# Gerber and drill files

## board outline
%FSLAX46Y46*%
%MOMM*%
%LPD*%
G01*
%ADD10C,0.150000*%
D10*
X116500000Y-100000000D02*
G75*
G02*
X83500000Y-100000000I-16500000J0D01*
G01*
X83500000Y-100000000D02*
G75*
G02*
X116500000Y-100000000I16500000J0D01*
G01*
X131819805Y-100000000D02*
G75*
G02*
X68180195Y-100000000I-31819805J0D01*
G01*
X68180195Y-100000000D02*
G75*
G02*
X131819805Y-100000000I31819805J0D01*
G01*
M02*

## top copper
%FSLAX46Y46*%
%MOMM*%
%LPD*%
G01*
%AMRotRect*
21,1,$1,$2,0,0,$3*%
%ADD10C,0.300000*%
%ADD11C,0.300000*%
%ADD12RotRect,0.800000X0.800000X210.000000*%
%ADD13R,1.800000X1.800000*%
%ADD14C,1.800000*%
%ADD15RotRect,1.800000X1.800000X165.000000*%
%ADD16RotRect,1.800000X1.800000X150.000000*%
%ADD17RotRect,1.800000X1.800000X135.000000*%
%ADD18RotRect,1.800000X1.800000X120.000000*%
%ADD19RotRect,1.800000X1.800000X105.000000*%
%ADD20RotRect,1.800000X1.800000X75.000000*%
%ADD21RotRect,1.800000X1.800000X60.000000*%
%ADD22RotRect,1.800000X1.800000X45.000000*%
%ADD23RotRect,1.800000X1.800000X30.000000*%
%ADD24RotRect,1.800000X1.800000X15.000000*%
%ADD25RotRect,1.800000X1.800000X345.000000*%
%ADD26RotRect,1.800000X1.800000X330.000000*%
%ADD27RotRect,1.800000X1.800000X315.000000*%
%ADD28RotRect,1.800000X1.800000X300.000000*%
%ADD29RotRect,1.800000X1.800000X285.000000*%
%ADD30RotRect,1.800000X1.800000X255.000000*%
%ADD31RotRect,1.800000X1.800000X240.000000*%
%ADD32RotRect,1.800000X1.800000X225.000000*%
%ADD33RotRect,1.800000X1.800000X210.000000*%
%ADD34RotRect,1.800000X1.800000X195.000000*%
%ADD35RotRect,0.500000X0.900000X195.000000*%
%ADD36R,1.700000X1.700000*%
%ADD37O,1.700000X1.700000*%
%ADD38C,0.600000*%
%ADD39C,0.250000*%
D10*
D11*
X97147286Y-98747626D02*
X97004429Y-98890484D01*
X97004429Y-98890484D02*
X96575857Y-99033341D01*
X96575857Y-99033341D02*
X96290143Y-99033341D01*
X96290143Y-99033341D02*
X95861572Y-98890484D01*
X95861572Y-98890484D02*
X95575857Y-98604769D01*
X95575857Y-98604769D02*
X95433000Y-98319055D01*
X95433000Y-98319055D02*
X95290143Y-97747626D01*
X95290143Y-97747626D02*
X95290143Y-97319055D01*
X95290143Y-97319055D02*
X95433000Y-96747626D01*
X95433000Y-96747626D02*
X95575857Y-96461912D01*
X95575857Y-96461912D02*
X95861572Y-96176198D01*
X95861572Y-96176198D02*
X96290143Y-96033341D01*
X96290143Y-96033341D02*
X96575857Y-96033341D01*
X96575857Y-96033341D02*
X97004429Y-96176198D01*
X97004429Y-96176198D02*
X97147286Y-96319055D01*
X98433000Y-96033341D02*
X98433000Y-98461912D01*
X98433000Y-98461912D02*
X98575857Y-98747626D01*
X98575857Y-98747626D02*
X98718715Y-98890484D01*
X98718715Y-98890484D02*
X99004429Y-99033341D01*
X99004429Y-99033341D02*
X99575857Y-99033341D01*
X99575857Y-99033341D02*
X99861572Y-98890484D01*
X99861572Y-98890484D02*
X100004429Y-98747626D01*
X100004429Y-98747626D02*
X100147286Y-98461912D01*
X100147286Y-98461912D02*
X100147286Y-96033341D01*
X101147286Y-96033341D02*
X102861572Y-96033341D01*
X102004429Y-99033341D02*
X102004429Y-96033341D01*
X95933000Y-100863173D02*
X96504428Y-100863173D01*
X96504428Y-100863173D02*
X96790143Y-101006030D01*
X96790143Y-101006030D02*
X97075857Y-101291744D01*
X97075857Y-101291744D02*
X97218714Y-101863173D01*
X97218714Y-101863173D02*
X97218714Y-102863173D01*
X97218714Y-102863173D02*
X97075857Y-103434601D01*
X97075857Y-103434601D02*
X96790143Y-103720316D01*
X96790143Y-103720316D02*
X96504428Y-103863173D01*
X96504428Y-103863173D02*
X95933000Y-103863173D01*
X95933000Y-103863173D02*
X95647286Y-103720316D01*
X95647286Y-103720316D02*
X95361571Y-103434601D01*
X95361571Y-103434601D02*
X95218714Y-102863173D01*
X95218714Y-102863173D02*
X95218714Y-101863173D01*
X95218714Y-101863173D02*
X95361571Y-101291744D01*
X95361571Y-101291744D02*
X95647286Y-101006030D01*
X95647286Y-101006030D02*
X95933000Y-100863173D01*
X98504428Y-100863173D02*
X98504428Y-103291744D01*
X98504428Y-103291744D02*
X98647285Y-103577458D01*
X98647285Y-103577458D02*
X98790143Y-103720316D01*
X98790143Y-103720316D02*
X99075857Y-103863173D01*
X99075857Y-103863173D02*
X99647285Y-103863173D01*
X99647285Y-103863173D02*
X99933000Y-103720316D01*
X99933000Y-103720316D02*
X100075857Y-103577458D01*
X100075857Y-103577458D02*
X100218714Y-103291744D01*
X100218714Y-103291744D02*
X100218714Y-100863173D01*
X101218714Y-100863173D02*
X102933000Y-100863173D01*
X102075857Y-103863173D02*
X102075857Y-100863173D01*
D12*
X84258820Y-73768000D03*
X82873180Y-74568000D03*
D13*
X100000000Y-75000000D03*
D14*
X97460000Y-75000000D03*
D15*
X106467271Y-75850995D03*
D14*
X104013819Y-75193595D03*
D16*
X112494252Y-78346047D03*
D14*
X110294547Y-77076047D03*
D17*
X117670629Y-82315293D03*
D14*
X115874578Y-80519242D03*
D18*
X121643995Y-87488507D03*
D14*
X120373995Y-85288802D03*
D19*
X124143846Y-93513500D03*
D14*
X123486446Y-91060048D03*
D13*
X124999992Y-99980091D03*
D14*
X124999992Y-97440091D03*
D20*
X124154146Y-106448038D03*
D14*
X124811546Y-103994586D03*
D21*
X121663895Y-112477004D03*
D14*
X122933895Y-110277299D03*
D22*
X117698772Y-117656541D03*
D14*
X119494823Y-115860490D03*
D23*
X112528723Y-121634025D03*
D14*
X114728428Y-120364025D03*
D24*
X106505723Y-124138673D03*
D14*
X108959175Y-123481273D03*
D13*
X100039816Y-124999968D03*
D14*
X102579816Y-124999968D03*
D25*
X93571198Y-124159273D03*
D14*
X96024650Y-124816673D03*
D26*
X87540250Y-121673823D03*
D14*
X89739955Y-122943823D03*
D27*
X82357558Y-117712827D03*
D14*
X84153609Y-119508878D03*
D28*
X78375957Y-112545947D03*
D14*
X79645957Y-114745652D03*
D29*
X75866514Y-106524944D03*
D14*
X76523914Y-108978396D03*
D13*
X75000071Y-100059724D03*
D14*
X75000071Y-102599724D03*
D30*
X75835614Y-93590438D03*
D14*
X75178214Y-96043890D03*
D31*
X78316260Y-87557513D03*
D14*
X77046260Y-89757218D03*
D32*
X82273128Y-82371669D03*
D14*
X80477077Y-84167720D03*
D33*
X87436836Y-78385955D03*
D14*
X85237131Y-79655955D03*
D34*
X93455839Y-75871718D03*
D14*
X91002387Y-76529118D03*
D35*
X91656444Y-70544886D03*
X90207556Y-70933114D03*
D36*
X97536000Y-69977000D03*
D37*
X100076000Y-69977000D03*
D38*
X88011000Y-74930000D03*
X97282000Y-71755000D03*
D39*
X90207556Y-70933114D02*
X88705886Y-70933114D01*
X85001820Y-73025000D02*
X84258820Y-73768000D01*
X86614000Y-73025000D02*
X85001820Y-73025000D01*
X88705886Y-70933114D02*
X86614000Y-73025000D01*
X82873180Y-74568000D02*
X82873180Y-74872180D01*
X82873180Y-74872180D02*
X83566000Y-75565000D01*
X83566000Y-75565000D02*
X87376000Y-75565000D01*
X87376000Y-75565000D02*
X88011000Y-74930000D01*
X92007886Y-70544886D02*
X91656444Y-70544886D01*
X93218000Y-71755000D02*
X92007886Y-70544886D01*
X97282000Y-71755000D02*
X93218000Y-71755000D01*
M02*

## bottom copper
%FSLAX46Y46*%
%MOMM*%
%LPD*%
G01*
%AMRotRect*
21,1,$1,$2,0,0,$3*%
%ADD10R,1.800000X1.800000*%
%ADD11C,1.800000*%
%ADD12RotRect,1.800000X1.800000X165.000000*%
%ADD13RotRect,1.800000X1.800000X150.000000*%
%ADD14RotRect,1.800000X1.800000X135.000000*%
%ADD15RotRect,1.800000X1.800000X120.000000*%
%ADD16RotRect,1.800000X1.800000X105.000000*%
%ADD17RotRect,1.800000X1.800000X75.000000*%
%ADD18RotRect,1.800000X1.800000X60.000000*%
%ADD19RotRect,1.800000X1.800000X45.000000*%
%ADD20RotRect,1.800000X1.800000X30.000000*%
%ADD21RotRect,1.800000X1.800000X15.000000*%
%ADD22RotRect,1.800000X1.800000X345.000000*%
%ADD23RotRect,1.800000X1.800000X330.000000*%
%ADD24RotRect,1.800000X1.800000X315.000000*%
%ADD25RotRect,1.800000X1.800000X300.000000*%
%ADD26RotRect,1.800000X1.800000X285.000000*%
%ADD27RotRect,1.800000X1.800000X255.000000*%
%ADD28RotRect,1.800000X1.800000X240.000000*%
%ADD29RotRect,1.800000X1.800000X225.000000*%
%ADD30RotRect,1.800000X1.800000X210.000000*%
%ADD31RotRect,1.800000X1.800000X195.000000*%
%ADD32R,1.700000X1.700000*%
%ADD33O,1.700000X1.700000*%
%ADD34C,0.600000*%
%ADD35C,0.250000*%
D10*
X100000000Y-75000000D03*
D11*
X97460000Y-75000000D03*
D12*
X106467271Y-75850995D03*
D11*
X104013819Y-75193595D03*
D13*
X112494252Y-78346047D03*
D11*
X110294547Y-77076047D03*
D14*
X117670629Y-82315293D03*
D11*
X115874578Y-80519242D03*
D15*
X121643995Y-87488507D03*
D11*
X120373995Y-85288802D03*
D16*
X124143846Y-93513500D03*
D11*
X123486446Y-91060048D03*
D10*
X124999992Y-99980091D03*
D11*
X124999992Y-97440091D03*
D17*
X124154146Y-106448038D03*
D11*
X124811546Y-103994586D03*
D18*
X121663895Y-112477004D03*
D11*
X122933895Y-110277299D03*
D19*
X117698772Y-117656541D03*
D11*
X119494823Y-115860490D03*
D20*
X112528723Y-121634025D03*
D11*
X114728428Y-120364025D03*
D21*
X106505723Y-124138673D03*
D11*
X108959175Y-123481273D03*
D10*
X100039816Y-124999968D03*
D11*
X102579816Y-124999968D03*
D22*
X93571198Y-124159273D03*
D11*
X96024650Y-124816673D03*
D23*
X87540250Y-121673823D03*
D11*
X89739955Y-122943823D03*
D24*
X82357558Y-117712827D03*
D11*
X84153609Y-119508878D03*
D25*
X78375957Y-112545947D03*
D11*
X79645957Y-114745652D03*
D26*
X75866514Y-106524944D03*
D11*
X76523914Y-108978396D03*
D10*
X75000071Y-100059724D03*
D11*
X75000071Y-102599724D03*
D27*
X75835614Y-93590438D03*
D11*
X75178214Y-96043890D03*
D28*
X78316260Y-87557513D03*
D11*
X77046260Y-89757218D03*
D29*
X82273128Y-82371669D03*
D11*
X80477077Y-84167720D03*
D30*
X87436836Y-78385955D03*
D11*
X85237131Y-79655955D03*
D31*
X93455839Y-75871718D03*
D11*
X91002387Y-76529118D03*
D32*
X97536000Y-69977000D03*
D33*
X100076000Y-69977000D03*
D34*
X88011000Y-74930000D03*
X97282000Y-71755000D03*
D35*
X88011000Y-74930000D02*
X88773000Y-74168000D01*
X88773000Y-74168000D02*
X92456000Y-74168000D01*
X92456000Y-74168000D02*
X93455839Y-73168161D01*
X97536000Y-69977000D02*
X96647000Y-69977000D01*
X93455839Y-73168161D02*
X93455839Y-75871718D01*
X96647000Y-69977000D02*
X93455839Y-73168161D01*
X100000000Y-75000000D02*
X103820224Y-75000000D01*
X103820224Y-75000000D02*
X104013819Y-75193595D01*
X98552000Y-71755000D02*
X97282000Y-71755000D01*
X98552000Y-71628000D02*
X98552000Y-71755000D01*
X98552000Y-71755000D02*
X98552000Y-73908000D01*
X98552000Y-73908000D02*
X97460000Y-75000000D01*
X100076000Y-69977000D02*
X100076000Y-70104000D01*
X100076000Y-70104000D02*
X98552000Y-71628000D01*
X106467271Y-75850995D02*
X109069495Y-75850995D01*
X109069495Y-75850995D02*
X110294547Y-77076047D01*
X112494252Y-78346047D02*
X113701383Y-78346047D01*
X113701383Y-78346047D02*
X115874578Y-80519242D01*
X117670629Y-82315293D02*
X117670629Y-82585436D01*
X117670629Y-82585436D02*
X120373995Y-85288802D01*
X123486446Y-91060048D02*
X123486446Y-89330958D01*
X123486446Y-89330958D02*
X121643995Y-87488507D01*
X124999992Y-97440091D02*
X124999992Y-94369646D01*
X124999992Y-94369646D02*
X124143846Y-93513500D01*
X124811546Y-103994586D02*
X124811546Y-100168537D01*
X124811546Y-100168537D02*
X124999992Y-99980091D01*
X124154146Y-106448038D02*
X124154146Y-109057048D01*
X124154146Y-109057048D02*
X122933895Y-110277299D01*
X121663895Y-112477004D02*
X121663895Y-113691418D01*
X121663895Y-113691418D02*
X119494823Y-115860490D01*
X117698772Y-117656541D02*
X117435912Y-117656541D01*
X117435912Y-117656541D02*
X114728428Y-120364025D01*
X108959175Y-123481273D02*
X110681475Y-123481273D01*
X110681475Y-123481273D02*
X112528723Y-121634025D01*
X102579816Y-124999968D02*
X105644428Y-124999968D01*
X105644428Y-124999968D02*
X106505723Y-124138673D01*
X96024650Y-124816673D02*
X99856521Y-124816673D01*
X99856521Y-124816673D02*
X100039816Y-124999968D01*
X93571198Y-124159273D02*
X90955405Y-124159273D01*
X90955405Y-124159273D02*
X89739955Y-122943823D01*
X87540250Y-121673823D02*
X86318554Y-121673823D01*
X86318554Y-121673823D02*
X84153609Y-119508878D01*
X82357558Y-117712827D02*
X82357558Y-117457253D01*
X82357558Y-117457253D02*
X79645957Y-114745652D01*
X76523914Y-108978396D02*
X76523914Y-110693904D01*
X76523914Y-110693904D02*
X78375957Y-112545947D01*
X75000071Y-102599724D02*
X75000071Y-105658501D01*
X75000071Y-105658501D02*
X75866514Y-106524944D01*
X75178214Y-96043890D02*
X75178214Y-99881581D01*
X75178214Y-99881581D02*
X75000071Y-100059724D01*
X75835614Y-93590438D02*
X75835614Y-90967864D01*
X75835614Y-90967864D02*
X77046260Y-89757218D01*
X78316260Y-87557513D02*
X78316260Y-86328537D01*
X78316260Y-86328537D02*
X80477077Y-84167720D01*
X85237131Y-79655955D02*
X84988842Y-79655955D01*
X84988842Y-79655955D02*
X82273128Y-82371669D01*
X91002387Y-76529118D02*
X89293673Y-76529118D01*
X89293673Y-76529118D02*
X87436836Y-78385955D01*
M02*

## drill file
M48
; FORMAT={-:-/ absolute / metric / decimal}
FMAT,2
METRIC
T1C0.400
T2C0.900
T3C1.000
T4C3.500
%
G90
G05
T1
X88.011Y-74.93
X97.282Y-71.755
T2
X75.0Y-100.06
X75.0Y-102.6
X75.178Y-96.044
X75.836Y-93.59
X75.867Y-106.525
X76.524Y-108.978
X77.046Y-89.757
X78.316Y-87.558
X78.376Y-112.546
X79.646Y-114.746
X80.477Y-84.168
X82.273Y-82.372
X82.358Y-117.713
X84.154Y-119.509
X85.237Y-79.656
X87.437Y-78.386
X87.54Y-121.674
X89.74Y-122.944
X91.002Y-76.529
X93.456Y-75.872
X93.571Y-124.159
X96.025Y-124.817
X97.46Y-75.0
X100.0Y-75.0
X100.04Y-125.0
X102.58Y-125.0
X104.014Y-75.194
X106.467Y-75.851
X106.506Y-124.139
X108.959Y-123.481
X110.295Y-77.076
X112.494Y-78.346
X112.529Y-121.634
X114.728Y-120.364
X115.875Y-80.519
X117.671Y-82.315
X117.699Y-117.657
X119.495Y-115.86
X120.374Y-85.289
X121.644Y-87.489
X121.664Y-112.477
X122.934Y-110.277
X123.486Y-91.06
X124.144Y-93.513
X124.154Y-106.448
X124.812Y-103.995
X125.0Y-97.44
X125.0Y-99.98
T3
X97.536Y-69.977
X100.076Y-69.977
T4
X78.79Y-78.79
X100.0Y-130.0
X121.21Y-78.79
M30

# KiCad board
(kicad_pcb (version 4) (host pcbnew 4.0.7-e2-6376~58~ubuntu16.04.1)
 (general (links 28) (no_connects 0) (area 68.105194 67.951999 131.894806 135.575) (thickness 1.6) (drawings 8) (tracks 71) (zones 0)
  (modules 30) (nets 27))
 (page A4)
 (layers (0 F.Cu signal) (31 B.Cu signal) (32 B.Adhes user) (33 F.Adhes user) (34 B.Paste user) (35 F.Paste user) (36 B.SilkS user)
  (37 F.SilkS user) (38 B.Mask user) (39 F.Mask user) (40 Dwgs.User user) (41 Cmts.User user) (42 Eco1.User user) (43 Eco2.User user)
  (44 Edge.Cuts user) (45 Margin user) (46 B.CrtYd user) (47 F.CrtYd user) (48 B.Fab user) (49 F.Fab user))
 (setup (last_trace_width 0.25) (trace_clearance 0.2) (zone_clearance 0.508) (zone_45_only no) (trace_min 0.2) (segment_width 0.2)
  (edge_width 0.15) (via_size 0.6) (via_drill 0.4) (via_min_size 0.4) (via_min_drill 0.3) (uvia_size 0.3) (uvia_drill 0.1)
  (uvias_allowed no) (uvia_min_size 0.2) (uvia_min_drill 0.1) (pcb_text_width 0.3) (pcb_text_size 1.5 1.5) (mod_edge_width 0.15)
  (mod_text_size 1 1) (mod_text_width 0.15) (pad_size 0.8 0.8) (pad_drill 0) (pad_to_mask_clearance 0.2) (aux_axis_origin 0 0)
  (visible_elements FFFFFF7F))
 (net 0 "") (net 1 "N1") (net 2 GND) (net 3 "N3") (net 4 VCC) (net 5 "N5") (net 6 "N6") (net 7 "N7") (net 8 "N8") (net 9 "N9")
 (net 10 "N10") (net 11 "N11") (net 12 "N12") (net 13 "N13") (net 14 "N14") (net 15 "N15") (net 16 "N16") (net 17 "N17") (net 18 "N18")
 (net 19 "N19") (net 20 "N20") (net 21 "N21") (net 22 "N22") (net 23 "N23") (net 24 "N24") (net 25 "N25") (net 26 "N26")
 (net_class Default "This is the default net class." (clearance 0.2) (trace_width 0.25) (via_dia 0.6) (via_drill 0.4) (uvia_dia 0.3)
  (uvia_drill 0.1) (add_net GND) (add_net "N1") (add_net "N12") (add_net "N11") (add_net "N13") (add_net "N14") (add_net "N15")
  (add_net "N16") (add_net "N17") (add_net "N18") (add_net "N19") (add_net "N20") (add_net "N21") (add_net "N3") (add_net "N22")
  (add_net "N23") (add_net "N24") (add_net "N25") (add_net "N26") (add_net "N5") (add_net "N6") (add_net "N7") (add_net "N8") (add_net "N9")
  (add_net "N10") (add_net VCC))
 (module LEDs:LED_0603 (layer F.Cu) (at 83.566 74.168 30)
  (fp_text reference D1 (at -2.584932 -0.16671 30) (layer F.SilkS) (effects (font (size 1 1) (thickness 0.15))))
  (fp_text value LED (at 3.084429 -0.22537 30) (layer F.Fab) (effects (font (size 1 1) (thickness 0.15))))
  (pad 2 smd rect (at 0.8 0 210) (size 0.8 0.8) (layers F.Cu F.Paste F.Mask) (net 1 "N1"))
  (pad 1 smd rect (at -0.8 0 210) (size 0.8 0.8) (layers F.Cu F.Paste F.Mask) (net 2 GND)))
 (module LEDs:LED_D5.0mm (layer F.Cu) (at 100 75 180)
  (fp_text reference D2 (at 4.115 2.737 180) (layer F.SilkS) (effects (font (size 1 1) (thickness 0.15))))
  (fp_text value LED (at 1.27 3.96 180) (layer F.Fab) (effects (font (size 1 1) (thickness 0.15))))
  (pad 1 thru_hole rect (at 0 0 180) (size 1.8 1.8) (drill 0.9) (layers *.Cu *.Mask) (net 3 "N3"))
  (pad 2 thru_hole circle (at 2.54 0 180) (size 1.8 1.8) (drill 0.9) (layers *.Cu *.Mask) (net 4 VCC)))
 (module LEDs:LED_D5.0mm (layer F.Cu) (at 106.467271 75.850995 165)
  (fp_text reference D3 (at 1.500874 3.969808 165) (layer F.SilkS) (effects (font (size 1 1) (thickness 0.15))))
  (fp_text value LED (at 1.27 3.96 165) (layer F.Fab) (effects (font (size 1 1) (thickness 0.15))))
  (pad 1 thru_hole rect (at 0 0 165) (size 1.8 1.8) (drill 0.9) (layers *.Cu *.Mask) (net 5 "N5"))
  (pad 2 thru_hole circle (at 2.54 0 165) (size 1.8 1.8) (drill 0.9) (layers *.Cu *.Mask) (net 3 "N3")))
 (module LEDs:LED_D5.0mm (layer F.Cu) (at 112.494252 78.346047 150)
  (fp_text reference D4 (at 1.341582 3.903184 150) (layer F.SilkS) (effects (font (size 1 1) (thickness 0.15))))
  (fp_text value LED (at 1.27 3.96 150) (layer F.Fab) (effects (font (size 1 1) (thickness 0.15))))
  (pad 1 thru_hole rect (at 0 0 150) (size 1.8 1.8) (drill 0.9) (layers *.Cu *.Mask) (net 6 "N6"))
  (pad 2 thru_hole circle (at 2.54 0 150) (size 1.8 1.8) (drill 0.9) (layers *.Cu *.Mask) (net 5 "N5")))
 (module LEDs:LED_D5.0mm (layer F.Cu) (at 117.670629 82.315293 135)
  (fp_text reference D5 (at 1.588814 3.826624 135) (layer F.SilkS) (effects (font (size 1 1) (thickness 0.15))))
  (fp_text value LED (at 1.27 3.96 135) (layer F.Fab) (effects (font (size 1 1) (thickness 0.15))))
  (pad 1 thru_hole rect (at 0 0 135) (size 1.8 1.8) (drill 0.9) (layers *.Cu *.Mask) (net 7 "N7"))
  (pad 2 thru_hole circle (at 2.54 0 135) (size 1.8 1.8) (drill 0.9) (layers *.Cu *.Mask) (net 6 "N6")))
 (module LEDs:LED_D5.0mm (layer F.Cu) (at 121.643995 87.488507 120)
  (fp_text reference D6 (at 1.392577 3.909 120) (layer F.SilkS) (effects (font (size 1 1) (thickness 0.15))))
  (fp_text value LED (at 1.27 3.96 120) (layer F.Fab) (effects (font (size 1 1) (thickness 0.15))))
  (pad 1 thru_hole rect (at 0 0 120) (size 1.8 1.8) (drill 0.9) (layers *.Cu *.Mask) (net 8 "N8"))
  (pad 2 thru_hole circle (at 2.54 0 120) (size 1.8 1.8) (drill 0.9) (layers *.Cu *.Mask) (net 7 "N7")))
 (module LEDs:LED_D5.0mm (layer F.Cu) (at 124.143846 93.5135 105)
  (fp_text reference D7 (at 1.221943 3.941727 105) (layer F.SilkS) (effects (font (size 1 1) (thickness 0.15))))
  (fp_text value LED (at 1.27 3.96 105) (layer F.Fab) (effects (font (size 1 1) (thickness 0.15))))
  (pad 1 thru_hole rect (at 0 0 105) (size 1.8 1.8) (drill 0.9) (layers *.Cu *.Mask) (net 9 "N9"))
  (pad 2 thru_hole circle (at 2.54 0 105) (size 1.8 1.8) (drill 0.9) (layers *.Cu *.Mask) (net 8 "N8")))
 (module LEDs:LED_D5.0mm (layer F.Cu) (at 124.999992 99.980091 90)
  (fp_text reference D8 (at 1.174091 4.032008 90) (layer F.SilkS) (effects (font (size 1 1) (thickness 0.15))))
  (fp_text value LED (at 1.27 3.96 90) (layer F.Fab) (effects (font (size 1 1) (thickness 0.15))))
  (pad 1 thru_hole rect (at 0 0 90) (size 1.8 1.8) (drill 0.9) (layers *.Cu *.Mask) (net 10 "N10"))
  (pad 2 thru_hole circle (at 2.54 0 90) (size 1.8 1.8) (drill 0.9) (layers *.Cu *.Mask) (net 9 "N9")))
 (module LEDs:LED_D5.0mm (layer F.Cu) (at 124.154146 106.448038 75)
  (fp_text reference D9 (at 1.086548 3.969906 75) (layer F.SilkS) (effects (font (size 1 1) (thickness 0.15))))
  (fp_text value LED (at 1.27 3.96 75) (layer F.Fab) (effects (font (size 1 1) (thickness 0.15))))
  (pad 1 thru_hole rect (at 0 0 75) (size 1.8 1.8) (drill 0.9) (layers *.Cu *.Mask) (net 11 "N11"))
  (pad 2 thru_hole circle (at 2.54 0 75) (size 1.8 1.8) (drill 0.9) (layers *.Cu *.Mask) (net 10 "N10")))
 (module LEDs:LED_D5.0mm (layer F.Cu) (at 121.663895 112.477004 60)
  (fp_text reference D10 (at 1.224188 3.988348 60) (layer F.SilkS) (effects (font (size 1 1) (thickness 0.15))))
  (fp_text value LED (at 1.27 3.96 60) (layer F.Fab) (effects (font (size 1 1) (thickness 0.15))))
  (pad 1 thru_hole rect (at 0 0 60) (size 1.8 1.8) (drill 0.9) (layers *.Cu *.Mask) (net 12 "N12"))
  (pad 2 thru_hole circle (at 2.54 0 60) (size 1.8 1.8) (drill 0.9) (layers *.Cu *.Mask) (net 11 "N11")))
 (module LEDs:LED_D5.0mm (layer F.Cu) (at 117.698772 117.656541 45)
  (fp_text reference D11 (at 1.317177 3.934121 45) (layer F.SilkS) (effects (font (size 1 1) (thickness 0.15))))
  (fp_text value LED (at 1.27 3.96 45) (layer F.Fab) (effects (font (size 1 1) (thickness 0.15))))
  (pad 1 thru_hole rect (at 0 0 45) (size 1.8 1.8) (drill 0.9) (layers *.Cu *.Mask) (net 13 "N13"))
  (pad 2 thru_hole circle (at 2.54 0 45) (size 1.8 1.8) (drill 0.9) (layers *.Cu *.Mask) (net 12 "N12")))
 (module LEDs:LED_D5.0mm (layer F.Cu) (at 112.528723 121.634025 30)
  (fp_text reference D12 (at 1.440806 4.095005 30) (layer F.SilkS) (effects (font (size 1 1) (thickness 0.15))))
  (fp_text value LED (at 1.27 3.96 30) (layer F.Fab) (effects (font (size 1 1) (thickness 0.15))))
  (pad 1 thru_hole rect (at 0 0 30) (size 1.8 1.8) (drill 0.9) (layers *.Cu *.Mask) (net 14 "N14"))
  (pad 2 thru_hole circle (at 2.54 0 30) (size 1.8 1.8) (drill 0.9) (layers *.Cu *.Mask) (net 13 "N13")))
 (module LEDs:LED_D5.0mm (layer F.Cu) (at 106.505723 124.138673 15)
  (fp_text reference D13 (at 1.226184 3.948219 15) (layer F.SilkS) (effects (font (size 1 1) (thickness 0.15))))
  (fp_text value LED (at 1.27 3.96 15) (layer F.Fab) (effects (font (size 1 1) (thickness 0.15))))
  (pad 1 thru_hole rect (at 0 0 15) (size 1.8 1.8) (drill 0.9) (layers *.Cu *.Mask) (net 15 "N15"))
  (pad 2 thru_hole circle (at 2.54 0 15) (size 1.8 1.8) (drill 0.9) (layers *.Cu *.Mask) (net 14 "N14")))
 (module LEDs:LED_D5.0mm (layer F.Cu) (at 100.039816 124.999968)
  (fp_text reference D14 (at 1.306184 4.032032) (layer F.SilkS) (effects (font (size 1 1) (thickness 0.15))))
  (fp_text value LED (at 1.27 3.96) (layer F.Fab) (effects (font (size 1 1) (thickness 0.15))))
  (pad 1 thru_hole rect (at 0 0) (size 1.8 1.8) (drill 0.9) (layers *.Cu *.Mask) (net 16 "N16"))
  (pad 2 thru_hole circle (at 2.54 0) (size 1.8 1.8) (drill 0.9) (layers *.Cu *.Mask) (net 15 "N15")))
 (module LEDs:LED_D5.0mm (layer F.Cu) (at 93.571198 124.159273 345)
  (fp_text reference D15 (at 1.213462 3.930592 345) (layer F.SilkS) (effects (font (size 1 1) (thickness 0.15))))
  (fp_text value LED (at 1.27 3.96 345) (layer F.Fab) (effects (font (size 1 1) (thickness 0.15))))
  (pad 1 thru_hole rect (at 0 0 345) (size 1.8 1.8) (drill 0.9) (layers *.Cu *.Mask) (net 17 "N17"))
  (pad 2 thru_hole circle (at 2.54 0 345) (size 1.8 1.8) (drill 0.9) (layers *.Cu *.Mask) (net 16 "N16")))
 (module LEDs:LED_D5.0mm (layer F.Cu) (at 87.54025 121.673823 330)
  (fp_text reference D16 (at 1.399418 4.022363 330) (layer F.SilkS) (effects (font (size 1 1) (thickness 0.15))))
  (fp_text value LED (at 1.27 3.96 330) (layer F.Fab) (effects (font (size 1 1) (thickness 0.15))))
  (pad 1 thru_hole rect (at 0 0 330) (size 1.8 1.8) (drill 0.9) (layers *.Cu *.Mask) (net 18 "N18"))
  (pad 2 thru_hole circle (at 2.54 0 330) (size 1.8 1.8) (drill 0.9) (layers *.Cu *.Mask) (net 17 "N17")))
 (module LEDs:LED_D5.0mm (layer F.Cu) (at 82.357558 117.712827 315)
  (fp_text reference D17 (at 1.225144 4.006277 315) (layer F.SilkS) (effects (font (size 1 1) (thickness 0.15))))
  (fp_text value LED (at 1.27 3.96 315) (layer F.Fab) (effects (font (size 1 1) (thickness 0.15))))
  (pad 1 thru_hole rect (at 0 0 315) (size 1.8 1.8) (drill 0.9) (layers *.Cu *.Mask) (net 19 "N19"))
  (pad 2 thru_hole circle (at 2.54 0 315) (size 1.8 1.8) (drill 0.9) (layers *.Cu *.Mask) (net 18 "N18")))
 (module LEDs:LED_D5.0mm (layer F.Cu) (at 78.375957 112.545947 300)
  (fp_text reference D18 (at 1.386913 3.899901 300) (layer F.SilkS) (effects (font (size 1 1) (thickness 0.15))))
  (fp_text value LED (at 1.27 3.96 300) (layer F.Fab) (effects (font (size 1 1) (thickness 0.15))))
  (pad 1 thru_hole rect (at 0 0 300) (size 1.8 1.8) (drill 0.9) (layers *.Cu *.Mask) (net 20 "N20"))
  (pad 2 thru_hole circle (at 2.54 0 300) (size 1.8 1.8) (drill 0.9) (layers *.Cu *.Mask) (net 19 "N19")))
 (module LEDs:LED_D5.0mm (layer F.Cu) (at 75.866514 106.524944 285)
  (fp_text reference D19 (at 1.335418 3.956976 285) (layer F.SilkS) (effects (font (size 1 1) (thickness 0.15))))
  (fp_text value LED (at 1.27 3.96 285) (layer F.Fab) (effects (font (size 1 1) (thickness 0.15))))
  (pad 1 thru_hole rect (at 0 0 285) (size 1.8 1.8) (drill 0.9) (layers *.Cu *.Mask) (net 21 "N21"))
  (pad 2 thru_hole circle (at 2.54 0 285) (size 1.8 1.8) (drill 0.9) (layers *.Cu *.Mask) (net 20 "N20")))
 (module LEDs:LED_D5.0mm (layer F.Cu) (at 75.000071 100.059724 270)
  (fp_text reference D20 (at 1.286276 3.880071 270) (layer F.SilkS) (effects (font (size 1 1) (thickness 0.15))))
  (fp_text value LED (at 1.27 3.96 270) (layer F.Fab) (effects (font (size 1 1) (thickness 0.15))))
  (pad 1 thru_hole rect (at 0 0 270) (size 1.8 1.8) (drill 0.9) (layers *.Cu *.Mask) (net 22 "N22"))
  (pad 2 thru_hole circle (at 2.54 0 270) (size 1.8 1.8) (drill 0.9) (layers *.Cu *.Mask) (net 21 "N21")))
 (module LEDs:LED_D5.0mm (layer F.Cu) (at 75.835614 93.590438 255)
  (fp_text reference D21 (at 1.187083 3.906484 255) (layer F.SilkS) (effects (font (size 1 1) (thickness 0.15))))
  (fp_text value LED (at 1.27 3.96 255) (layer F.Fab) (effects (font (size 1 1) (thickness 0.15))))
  (pad 1 thru_hole rect (at 0 0 255) (size 1.8 1.8) (drill 0.9) (layers *.Cu *.Mask) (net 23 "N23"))
  (pad 2 thru_hole circle (at 2.54 0 255) (size 1.8 1.8) (drill 0.9) (layers *.Cu *.Mask) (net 22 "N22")))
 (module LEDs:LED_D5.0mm (layer F.Cu) (at 78.31626 87.557513 240)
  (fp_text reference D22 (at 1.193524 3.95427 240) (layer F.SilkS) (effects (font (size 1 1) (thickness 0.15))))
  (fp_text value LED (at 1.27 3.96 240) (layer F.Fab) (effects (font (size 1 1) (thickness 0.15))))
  (pad 1 thru_hole rect (at 0 0 240) (size 1.8 1.8) (drill 0.9) (layers *.Cu *.Mask) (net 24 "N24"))
  (pad 2 thru_hole circle (at 2.54 0 240) (size 1.8 1.8) (drill 0.9) (layers *.Cu *.Mask) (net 23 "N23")))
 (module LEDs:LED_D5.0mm (layer F.Cu) (at 82.273128 82.371669 225)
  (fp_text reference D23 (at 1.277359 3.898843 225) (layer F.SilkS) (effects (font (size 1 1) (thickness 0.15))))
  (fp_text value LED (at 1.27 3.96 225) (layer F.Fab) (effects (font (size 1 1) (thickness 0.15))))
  (pad 1 thru_hole rect (at 0 0 225) (size 1.8 1.8) (drill 0.9) (layers *.Cu *.Mask) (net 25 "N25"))
  (pad 2 thru_hole circle (at 2.54 0 225) (size 1.8 1.8) (drill 0.9) (layers *.Cu *.Mask) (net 24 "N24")))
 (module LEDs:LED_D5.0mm (layer F.Cu) (at 87.436836 78.385955 210)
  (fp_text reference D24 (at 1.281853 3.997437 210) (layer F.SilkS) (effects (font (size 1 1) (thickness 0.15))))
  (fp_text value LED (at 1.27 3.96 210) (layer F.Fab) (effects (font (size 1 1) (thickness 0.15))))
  (pad 1 thru_hole rect (at 0 0 210) (size 1.8 1.8) (drill 0.9) (layers *.Cu *.Mask) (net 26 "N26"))
  (pad 2 thru_hole circle (at 2.54 0 210) (size 1.8 1.8) (drill 0.9) (layers *.Cu *.Mask) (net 25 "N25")))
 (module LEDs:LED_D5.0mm (layer F.Cu) (at 93.455839 75.871718 195)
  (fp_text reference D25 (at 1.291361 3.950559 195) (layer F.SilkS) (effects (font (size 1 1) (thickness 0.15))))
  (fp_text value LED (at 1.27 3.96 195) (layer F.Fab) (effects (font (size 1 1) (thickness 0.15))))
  (pad 1 thru_hole rect (at 0 0 195) (size 1.8 1.8) (drill 0.9) (layers *.Cu *.Mask) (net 2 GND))
  (pad 2 thru_hole circle (at 2.54 0 195) (size 1.8 1.8) (drill 0.9) (layers *.Cu *.Mask) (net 26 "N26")))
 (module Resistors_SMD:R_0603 (layer F.Cu) (at 90.932 70.739 195)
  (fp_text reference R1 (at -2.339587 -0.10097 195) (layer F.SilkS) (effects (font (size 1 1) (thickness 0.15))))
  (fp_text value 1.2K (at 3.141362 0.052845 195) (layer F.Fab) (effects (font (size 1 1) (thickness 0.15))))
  (pad 1 smd rect (at -0.75 0 195) (size 0.5 0.9) (layers F.Cu F.Paste F.Mask) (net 4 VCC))
  (pad 2 smd rect (at 0.75 0 195) (size 0.5 0.9) (layers F.Cu F.Paste F.Mask) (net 1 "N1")))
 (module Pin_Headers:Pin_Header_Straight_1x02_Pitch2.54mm (layer F.Cu) (at 97.536 69.977 90)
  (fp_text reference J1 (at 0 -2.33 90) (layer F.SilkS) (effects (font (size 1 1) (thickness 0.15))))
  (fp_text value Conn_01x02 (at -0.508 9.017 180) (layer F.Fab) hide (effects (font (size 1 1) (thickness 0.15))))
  (pad 1 thru_hole rect (at 0 0 90) (size 1.7 1.7) (drill 1) (layers *.Cu *.Mask) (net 2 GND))
  (pad 2 thru_hole oval (at 0 2.54 90) (size 1.7 1.7) (drill 1) (layers *.Cu *.Mask) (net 4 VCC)))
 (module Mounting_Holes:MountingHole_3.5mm (layer F.Cu) (at 100 130)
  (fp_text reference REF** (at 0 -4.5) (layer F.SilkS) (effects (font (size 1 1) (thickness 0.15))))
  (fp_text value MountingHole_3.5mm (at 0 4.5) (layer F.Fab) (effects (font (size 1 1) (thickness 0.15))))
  (pad 1 np_thru_hole circle (at 0 0) (size 3.5 3.5) (drill 3.5) (layers *.Cu *.Mask)))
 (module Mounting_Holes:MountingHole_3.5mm (layer F.Cu) (at 121.21 78.79)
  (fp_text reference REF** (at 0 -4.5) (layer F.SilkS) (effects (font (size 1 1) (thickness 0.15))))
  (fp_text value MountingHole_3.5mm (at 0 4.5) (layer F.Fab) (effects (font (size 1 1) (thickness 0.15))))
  (pad 1 np_thru_hole circle (at 0 0) (size 3.5 3.5) (drill 3.5) (layers *.Cu *.Mask)))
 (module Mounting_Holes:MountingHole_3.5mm (layer F.Cu) (at 78.79 78.79)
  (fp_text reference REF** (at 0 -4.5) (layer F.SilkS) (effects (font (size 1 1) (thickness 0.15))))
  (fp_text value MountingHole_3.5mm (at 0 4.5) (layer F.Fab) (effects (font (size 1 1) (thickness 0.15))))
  (pad 1 np_thru_hole circle (at 0 0) (size 3.5 3.5) (drill 3.5) (layers *.Cu *.Mask)))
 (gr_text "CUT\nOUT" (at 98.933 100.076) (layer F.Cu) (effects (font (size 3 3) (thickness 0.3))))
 (gr_circle (center 100 100) (end 116.5 100) (layer Edge.Cuts) (width 0.15))
 (gr_circle (center 100 100) (end 122.5 122.5) (layer Edge.Cuts) (width 0.15))
 (segment (start 90.207556 70.933114) (end 88.705886 70.933114) (width 0.25) (layer F.Cu) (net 1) (status 10))
 (segment (start 85.00182 73.025) (end 84.25882 73.768) (width 0.25) (layer F.Cu) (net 1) (status 20))
 (segment (start 86.614 73.025) (end 85.00182 73.025) (width 0.25) (layer F.Cu) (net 1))
 (segment (start 88.705886 70.933114) (end 86.614 73.025) (width 0.25) (layer F.Cu) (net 1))
 (segment (start 82.87318 74.568) (end 82.87318 74.87218) (width 0.25) (layer F.Cu) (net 2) (status 30))
 (segment (start 82.87318 74.87218) (end 83.566 75.565) (width 0.25) (layer F.Cu) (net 2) (status 10))
 (segment (start 83.566 75.565) (end 87.376 75.565) (width 0.25) (layer F.Cu) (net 2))
 (segment (start 87.376 75.565) (end 88.011 74.93) (width 0.25) (layer F.Cu) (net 2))
 (via (at 88.011 74.93) (size 0.6) (drill 0.4) (layers F.Cu B.Cu) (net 2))
 (segment (start 88.011 74.93) (end 88.773 74.168) (width 0.25) (layer B.Cu) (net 2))
 (segment (start 88.773 74.168) (end 92.456 74.168) (width 0.25) (layer B.Cu) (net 2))
 (segment (start 92.456 74.168) (end 93.455839 73.168161) (width 0.25) (layer B.Cu) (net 2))
 (segment (start 97.536 69.977) (end 96.647 69.977) (width 0.25) (layer B.Cu) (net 2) (status 10))
 (segment (start 93.455839 73.168161) (end 93.455839 75.871718) (width 0.25) (layer B.Cu) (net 2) (status 20))
 (segment (start 96.647 69.977) (end 93.455839 73.168161) (width 0.25) (layer B.Cu) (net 2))
 (segment (start 100 75) (end 103.820224 75) (width 0.25) (layer B.Cu) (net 3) (status 30))
 (segment (start 103.820224 75) (end 104.013819 75.193595) (width 0.25) (layer B.Cu) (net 3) (status 30))
 (segment (start 98.552 71.755) (end 97.282 71.755) (width 0.25) (layer B.Cu) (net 4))
 (segment (start 92.007886 70.544886) (end 91.656444 70.544886) (width 0.25) (layer F.Cu) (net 4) (status 20))
 (segment (start 93.218 71.755) (end 92.007886 70.544886) (width 0.25) (layer F.Cu) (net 4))
 (segment (start 97.282 71.755) (end 93.218 71.755) (width 0.25) (layer F.Cu) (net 4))
 (via (at 97.282 71.755) (size 0.6) (drill 0.4) (layers F.Cu B.Cu) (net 4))
 (segment (start 98.552 71.628) (end 98.552 71.755) (width 0.25) (layer B.Cu) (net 4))
 (segment (start 98.552 71.755) (end 98.552 73.908) (width 0.25) (layer B.Cu) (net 4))
 (segment (start 98.552 73.908) (end 97.46 75) (width 0.25) (layer B.Cu) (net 4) (status 20))
 (segment (start 100.076 69.977) (end 100.076 70.104) (width 0.25) (layer B.Cu) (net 4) (status 30))
 (segment (start 100.076 70.104) (end 98.552 71.628) (width 0.25) (layer B.Cu) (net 4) (status 10))
 (segment (start 106.467271 75.850995) (end 109.069495 75.850995) (width 0.25) (layer B.Cu) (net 5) (status 10))
 (segment (start 109.069495 75.850995) (end 110.294547 77.076047) (width 0.25) (layer B.Cu) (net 5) (status 20))
 (segment (start 112.494252 78.346047) (end 113.701383 78.346047) (width 0.25) (layer B.Cu) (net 6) (status 10))
 (segment (start 113.701383 78.346047) (end 115.874578 80.519242) (width 0.25) (layer B.Cu) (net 6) (status 20))
 (segment (start 117.670629 82.315293) (end 117.670629 82.585436) (width 0.25) (layer B.Cu) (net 7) (status 30))
 (segment (start 117.670629 82.585436) (end 120.373995 85.288802) (width 0.25) (layer B.Cu) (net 7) (status 30))
 (segment (start 123.486446 91.060048) (end 123.486446 89.330958) (width 0.25) (layer B.Cu) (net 8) (status 10))
 (segment (start 123.486446 89.330958) (end 121.643995 87.488507) (width 0.25) (layer B.Cu) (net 8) (status 20))
 (segment (start 124.999992 97.440091) (end 124.999992 94.369646) (width 0.25) (layer B.Cu) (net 9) (status 10))
 (segment (start 124.999992 94.369646) (end 124.143846 93.5135) (width 0.25) (layer B.Cu) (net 9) (status 20))
 (segment (start 124.811546 103.994586) (end 124.811546 100.168537) (width 0.25) (layer B.Cu) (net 10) (status 30))
 (segment (start 124.811546 100.168537) (end 124.999992 99.980091) (width 0.25) (layer B.Cu) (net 10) (status 30))
 (segment (start 124.154146 106.448038) (end 124.154146 109.057048) (width 0.25) (layer B.Cu) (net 11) (status 10))
 (segment (start 124.154146 109.057048) (end 122.933895 110.277299) (width 0.25) (layer B.Cu) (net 11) (status 20))
 (segment (start 121.663895 112.477004) (end 121.663895 113.691418) (width 0.25) (layer B.Cu) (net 12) (status 10))
 (segment (start 121.663895 113.691418) (end 119.494823 115.86049) (width 0.25) (layer B.Cu) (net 12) (status 20))
 (segment (start 117.698772 117.656541) (end 117.435912 117.656541) (width 0.25) (layer B.Cu) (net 13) (status 30))
 (segment (start 117.435912 117.656541) (end 114.728428 120.364025) (width 0.25) (layer B.Cu) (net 13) (status 30))
 (segment (start 108.959175 123.481273) (end 110.681475 123.481273) (width 0.25) (layer B.Cu) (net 14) (status 10))
 (segment (start 110.681475 123.481273) (end 112.528723 121.634025) (width 0.25) (layer B.Cu) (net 14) (status 20))
 (segment (start 102.579816 124.999968) (end 105.644428 124.999968) (width 0.25) (layer B.Cu) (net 15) (status 10))
 (segment (start 105.644428 124.999968) (end 106.505723 124.138673) (width 0.25) (layer B.Cu) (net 15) (status 20))
 (segment (start 96.02465 124.816673) (end 99.856521 124.816673) (width 0.25) (layer B.Cu) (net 16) (status 30))
 (segment (start 99.856521 124.816673) (end 100.039816 124.999968) (width 0.25) (layer B.Cu) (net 16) (status 30))
 (segment (start 93.571198 124.159273) (end 90.955405 124.159273) (width 0.25) (layer B.Cu) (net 17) (status 10))
 (segment (start 90.955405 124.159273) (end 89.739955 122.943823) (width 0.25) (layer B.Cu) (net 17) (status 20))
 (segment (start 87.54025 121.673823) (end 86.318554 121.673823) (width 0.25) (layer B.Cu) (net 18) (status 10))
 (segment (start 86.318554 121.673823) (end 84.153609 119.508878) (width 0.25) (layer B.Cu) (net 18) (status 20))
 (segment (start 82.357558 117.712827) (end 82.357558 117.457253) (width 0.25) (layer B.Cu) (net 19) (status 30))
 (segment (start 82.357558 117.457253) (end 79.645957 114.745652) (width 0.25) (layer B.Cu) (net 19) (status 30))
 (segment (start 76.523914 108.978396) (end 76.523914 110.693904) (width 0.25) (layer B.Cu) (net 20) (status 10))
 (segment (start 76.523914 110.693904) (end 78.375957 112.545947) (width 0.25) (layer B.Cu) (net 20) (status 20))
 (segment (start 75.000071 102.599724) (end 75.000071 105.658501) (width 0.25) (layer B.Cu) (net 21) (status 10))
 (segment (start 75.000071 105.658501) (end 75.866514 106.524944) (width 0.25) (layer B.Cu) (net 21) (status 20))
 (segment (start 75.178214 96.04389) (end 75.178214 99.881581) (width 0.25) (layer B.Cu) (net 22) (status 30))
 (segment (start 75.178214 99.881581) (end 75.000071 100.059724) (width 0.25) (layer B.Cu) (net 22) (status 30))
 (segment (start 75.835614 93.590438) (end 75.835614 90.967864) (width 0.25) (layer B.Cu) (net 23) (status 10))
 (segment (start 75.835614 90.967864) (end 77.04626 89.757218) (width 0.25) (layer B.Cu) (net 23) (status 20))
 (segment (start 78.31626 87.557513) (end 78.31626 86.328537) (width 0.25) (layer B.Cu) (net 24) (status 10))
 (segment (start 78.31626 86.328537) (end 80.477077 84.16772) (width 0.25) (layer B.Cu) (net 24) (status 20))
 (segment (start 85.237131 79.655955) (end 84.988842 79.655955) (width 0.25) (layer B.Cu) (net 25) (status 30))
 (segment (start 84.988842 79.655955) (end 82.273128 82.371669) (width 0.25) (layer B.Cu) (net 25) (status 30))
 (segment (start 91.002387 76.529118) (end 89.293673 76.529118) (width 0.25) (layer B.Cu) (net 26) (status 10))
 (segment (start 89.293673 76.529118) (end 87.436836 78.385955) (width 0.25) (layer B.Cu) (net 26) (status 20)))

